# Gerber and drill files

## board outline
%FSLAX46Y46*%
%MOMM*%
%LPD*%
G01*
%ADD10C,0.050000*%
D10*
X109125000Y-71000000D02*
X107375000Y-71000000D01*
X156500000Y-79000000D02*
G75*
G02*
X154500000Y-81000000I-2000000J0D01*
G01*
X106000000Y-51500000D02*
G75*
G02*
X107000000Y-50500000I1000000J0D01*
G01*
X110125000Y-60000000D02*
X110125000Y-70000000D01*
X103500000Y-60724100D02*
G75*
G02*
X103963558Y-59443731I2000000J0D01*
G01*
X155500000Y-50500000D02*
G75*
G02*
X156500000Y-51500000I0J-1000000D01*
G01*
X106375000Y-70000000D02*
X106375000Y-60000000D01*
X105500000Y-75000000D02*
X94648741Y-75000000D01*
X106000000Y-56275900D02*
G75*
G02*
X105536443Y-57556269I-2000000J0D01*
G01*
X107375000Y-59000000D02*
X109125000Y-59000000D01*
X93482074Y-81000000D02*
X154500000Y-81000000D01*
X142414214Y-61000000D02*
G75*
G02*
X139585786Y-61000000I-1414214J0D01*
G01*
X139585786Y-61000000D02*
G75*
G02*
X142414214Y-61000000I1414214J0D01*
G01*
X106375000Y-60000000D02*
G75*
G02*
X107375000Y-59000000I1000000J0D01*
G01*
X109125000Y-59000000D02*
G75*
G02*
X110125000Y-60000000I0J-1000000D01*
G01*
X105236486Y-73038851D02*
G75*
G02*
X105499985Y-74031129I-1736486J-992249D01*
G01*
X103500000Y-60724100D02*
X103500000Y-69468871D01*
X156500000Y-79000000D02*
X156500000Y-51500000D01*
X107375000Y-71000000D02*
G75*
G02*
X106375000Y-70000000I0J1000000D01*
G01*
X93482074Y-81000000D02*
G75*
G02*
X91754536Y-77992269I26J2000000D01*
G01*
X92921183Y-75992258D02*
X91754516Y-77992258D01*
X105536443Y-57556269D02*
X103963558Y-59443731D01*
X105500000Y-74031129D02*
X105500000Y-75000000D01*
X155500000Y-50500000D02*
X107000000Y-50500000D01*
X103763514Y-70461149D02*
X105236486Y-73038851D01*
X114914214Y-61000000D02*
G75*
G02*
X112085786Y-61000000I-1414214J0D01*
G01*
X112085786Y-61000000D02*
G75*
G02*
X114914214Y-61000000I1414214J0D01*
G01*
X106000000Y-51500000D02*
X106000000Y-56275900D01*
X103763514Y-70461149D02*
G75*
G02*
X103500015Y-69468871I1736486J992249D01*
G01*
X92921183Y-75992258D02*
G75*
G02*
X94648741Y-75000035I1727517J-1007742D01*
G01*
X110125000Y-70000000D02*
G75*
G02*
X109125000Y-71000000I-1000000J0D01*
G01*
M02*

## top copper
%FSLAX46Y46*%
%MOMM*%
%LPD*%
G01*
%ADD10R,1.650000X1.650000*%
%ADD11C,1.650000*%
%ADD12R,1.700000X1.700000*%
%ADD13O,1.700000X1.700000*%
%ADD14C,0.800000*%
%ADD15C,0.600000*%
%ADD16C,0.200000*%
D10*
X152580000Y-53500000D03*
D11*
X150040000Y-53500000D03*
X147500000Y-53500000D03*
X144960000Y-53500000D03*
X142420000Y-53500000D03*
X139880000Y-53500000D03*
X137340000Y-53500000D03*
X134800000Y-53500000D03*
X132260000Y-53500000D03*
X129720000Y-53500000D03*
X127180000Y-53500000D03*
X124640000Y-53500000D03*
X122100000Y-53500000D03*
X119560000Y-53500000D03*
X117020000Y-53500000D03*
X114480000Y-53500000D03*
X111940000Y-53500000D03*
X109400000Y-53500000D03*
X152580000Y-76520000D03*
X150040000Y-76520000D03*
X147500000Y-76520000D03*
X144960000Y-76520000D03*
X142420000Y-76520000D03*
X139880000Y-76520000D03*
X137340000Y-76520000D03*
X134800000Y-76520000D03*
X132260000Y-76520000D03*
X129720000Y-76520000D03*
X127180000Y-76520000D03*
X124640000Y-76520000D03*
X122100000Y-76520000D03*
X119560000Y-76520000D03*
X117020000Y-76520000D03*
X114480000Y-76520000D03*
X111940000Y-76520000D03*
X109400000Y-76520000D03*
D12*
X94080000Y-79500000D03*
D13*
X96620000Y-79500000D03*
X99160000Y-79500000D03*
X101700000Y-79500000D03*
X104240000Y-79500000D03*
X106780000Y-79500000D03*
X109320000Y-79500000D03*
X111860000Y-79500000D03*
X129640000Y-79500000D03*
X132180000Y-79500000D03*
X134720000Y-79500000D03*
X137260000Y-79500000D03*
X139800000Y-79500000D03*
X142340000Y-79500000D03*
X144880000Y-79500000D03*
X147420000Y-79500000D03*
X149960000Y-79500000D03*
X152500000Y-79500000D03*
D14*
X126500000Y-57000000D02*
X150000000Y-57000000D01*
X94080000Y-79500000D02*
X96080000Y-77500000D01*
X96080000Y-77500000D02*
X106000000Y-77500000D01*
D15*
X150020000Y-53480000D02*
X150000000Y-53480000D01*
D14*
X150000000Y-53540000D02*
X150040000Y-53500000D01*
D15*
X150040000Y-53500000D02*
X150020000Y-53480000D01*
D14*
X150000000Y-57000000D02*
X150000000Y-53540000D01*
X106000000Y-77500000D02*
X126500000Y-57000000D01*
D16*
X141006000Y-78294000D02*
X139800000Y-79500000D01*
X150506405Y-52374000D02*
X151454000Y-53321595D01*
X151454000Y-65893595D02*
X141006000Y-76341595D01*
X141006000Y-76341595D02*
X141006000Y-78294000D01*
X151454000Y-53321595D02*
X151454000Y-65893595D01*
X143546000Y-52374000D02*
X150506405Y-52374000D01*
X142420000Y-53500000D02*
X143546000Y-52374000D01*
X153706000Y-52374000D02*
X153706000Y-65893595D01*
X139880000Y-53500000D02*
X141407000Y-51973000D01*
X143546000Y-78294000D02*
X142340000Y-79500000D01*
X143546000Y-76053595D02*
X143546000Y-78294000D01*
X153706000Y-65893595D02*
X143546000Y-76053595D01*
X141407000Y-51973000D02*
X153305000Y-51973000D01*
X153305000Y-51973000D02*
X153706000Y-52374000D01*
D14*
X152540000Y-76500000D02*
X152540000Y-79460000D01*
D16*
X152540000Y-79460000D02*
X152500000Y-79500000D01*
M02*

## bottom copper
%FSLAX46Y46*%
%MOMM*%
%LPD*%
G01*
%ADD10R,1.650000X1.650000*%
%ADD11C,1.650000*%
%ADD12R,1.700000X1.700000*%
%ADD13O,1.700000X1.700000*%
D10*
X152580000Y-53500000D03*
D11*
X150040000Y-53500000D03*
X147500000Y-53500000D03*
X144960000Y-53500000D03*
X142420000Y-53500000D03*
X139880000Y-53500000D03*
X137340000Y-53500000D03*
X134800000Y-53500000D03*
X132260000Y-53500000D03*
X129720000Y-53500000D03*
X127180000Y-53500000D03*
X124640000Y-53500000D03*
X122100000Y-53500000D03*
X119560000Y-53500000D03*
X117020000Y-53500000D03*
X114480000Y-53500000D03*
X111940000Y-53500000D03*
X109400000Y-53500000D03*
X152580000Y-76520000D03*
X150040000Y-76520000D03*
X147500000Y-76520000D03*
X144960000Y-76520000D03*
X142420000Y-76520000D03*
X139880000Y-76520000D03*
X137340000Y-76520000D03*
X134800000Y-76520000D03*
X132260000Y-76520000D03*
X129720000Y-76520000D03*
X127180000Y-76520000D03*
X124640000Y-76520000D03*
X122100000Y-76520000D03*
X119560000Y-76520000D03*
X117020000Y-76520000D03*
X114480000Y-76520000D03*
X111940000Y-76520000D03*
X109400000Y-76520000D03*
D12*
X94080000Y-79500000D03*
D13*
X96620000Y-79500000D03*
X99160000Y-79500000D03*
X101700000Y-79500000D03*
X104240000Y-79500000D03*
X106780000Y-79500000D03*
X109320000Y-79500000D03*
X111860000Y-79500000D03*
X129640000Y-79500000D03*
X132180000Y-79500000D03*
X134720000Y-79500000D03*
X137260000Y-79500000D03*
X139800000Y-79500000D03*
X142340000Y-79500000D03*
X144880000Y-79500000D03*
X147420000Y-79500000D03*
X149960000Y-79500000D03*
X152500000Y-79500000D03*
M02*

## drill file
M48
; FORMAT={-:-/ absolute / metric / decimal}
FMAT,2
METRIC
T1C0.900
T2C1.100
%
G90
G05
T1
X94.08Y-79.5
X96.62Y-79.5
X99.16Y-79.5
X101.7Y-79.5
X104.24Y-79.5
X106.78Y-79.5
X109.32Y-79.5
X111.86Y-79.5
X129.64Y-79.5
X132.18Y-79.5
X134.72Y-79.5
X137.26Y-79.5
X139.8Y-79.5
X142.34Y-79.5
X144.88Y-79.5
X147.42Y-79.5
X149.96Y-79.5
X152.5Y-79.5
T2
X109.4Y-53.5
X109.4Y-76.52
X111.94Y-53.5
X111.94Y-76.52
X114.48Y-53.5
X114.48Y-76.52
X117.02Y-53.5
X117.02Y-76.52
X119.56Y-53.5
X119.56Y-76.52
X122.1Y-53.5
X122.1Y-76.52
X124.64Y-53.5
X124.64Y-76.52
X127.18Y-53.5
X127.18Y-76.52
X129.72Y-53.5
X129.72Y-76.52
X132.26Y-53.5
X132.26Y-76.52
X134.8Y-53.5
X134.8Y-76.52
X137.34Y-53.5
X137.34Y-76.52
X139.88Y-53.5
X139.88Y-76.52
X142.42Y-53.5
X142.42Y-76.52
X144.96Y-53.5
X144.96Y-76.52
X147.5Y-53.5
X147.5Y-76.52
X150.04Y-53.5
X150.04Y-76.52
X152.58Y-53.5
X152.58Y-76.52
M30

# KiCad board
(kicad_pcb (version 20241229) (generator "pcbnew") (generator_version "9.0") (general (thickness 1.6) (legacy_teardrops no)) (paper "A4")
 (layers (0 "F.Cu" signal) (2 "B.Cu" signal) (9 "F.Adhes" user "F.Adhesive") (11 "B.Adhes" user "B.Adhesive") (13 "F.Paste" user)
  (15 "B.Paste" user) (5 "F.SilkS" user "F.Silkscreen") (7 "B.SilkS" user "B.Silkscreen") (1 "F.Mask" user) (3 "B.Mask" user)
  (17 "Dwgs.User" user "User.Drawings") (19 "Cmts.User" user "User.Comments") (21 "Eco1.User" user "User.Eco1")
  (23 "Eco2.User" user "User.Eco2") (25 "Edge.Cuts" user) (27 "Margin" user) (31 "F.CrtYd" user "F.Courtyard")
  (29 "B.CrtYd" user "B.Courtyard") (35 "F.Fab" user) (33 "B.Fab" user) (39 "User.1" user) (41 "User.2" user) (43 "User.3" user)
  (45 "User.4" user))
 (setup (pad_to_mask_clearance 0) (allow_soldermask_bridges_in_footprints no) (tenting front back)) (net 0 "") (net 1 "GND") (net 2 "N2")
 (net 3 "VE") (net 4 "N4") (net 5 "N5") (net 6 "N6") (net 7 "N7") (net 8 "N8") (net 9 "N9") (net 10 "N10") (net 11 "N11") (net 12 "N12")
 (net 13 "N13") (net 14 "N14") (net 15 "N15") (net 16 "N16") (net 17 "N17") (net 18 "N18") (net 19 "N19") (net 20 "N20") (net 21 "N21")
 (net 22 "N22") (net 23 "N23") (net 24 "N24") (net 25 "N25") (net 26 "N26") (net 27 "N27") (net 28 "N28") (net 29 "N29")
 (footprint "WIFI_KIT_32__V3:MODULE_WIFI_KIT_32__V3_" (layer "F.Cu") (at 130.18 65.01 -90)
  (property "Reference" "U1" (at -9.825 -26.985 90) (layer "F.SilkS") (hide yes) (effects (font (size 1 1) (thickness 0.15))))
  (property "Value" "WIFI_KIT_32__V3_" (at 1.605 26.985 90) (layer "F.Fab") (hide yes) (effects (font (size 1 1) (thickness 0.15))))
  (pad "J2_1" thru_hole rect (at -11.51 -22.4 270) (size 1.65 1.65) (drill 1.1) (layers "*.Cu" "*.Mask") (remove_unused_layers no)
   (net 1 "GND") (solder_mask_margin 0.102))
  (pad "J2_2" thru_hole circle (at -11.51 -19.86 270) (size 1.65 1.65) (drill 1.1) (layers "*.Cu" "*.Mask") (remove_unused_layers no)
   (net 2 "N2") (solder_mask_margin 0.102))
  (pad "J2_3" thru_hole circle (at -11.51 -17.32 270) (size 1.65 1.65) (drill 1.1) (layers "*.Cu" "*.Mask") (remove_unused_layers no)
   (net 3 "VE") (solder_mask_margin 0.102))
  (pad "J2_4" thru_hole circle (at -11.51 -14.78 270) (size 1.65 1.65) (drill 1.1) (layers "*.Cu" "*.Mask") (remove_unused_layers no)
   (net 3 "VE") (solder_mask_margin 0.102))
  (pad "J2_5" thru_hole circle (at -11.51 -12.24 270) (size 1.65 1.65) (drill 1.1) (layers "*.Cu" "*.Mask") (remove_unused_layers no)
   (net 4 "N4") (solder_mask_margin 0.102))
  (pad "J2_6" thru_hole circle (at -11.51 -9.7 270) (size 1.65 1.65) (drill 1.1) (layers "*.Cu" "*.Mask") (remove_unused_layers no)
   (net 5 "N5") (solder_mask_margin 0.102))
  (pad "J2_7" thru_hole circle (at -11.51 -7.16 270) (size 1.65 1.65) (drill 1.1) (layers "*.Cu" "*.Mask") (remove_unused_layers no)
   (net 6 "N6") (solder_mask_margin 0.102))
  (pad "J2_8" thru_hole circle (at -11.51 -4.62 270) (size 1.65 1.65) (drill 1.1) (layers "*.Cu" "*.Mask") (remove_unused_layers no)
   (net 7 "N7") (solder_mask_margin 0.102))
  (pad "J2_9" thru_hole circle (at -11.51 -2.08 270) (size 1.65 1.65) (drill 1.1) (layers "*.Cu" "*.Mask") (remove_unused_layers no)
   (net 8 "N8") (solder_mask_margin 0.102))
  (pad "J2_10" thru_hole circle (at -11.51 0.46 270) (size 1.65 1.65) (drill 1.1) (layers "*.Cu" "*.Mask") (remove_unused_layers no)
   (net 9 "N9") (solder_mask_margin 0.102))
  (pad "J2_11" thru_hole circle (at -11.51 3 270) (size 1.65 1.65) (drill 1.1) (layers "*.Cu" "*.Mask") (remove_unused_layers no)
   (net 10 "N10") (solder_mask_margin 0.102))
  (pad "J2_12" thru_hole circle (at -11.51 5.54 270) (size 1.65 1.65) (drill 1.1) (layers "*.Cu" "*.Mask") (remove_unused_layers no)
   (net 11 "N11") (solder_mask_margin 0.102))
  (pad "J2_13" thru_hole circle (at -11.51 8.08 270) (size 1.65 1.65) (drill 1.1) (layers "*.Cu" "*.Mask") (remove_unused_layers no)
   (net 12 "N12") (solder_mask_margin 0.102))
  (pad "J2_14" thru_hole circle (at -11.51 10.62 270) (size 1.65 1.65) (drill 1.1) (layers "*.Cu" "*.Mask") (remove_unused_layers no)
   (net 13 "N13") (solder_mask_margin 0.102))
  (pad "J2_15" thru_hole circle (at -11.51 13.16 270) (size 1.65 1.65) (drill 1.1) (layers "*.Cu" "*.Mask") (remove_unused_layers no)
   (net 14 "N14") (solder_mask_margin 0.102))
  (pad "J2_16" thru_hole circle (at -11.51 15.7 270) (size 1.65 1.65) (drill 1.1) (layers "*.Cu" "*.Mask") (remove_unused_layers no)
   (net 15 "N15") (solder_mask_margin 0.102))
  (pad "J2_17" thru_hole circle (at -11.51 18.24 270) (size 1.65 1.65) (drill 1.1) (layers "*.Cu" "*.Mask") (remove_unused_layers no)
   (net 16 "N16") (solder_mask_margin 0.102))
  (pad "J2_18" thru_hole circle (at -11.51 20.78 270) (size 1.65 1.65) (drill 1.1) (layers "*.Cu" "*.Mask") (remove_unused_layers no)
   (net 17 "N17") (solder_mask_margin 0.102))
  (pad "J3_1" thru_hole circle (at 11.51 -22.4 270) (size 1.65 1.65) (drill 1.1) (layers "*.Cu" "*.Mask") (remove_unused_layers no)
   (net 1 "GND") (solder_mask_margin 0.102))
  (pad "J3_2" thru_hole circle (at 11.51 -19.86 270) (size 1.65 1.65) (drill 1.1) (layers "*.Cu" "*.Mask") (remove_unused_layers no)
   (solder_mask_margin 0.102))
  (pad "J3_3" thru_hole circle (at 11.51 -17.32 270) (size 1.65 1.65) (drill 1.1) (layers "*.Cu" "*.Mask") (remove_unused_layers no)
   (solder_mask_margin 0.102))
  (pad "J3_4" thru_hole circle (at 11.51 -14.78 270) (size 1.65 1.65) (drill 1.1) (layers "*.Cu" "*.Mask") (remove_unused_layers no)
   (solder_mask_margin 0.102))
  (pad "J3_5" thru_hole circle (at 11.51 -12.24 270) (size 1.65 1.65) (drill 1.1) (layers "*.Cu" "*.Mask") (remove_unused_layers no)
   (solder_mask_margin 0.102))
  (pad "J3_6" thru_hole circle (at 11.51 -9.7 270) (size 1.65 1.65) (drill 1.1) (layers "*.Cu" "*.Mask") (remove_unused_layers no)
   (solder_mask_margin 0.102))
  (pad "J3_7" thru_hole circle (at 11.51 -7.16 270) (size 1.65 1.65) (drill 1.1) (layers "*.Cu" "*.Mask") (remove_unused_layers no)
   (solder_mask_margin 0.102))
  (pad "J3_8" thru_hole circle (at 11.51 -4.62 270) (size 1.65 1.65) (drill 1.1) (layers "*.Cu" "*.Mask") (remove_unused_layers no)
   (solder_mask_margin 0.102))
  (pad "J3_9" thru_hole circle (at 11.51 -2.08 270) (size 1.65 1.65) (drill 1.1) (layers "*.Cu" "*.Mask") (remove_unused_layers no)
   (solder_mask_margin 0.102))
  (pad "J3_10" thru_hole circle (at 11.51 0.46 270) (size 1.65 1.65) (drill 1.1) (layers "*.Cu" "*.Mask") (remove_unused_layers no)
   (solder_mask_margin 0.102))
  (pad "J3_11" thru_hole circle (at 11.51 3 270) (size 1.65 1.65) (drill 1.1) (layers "*.Cu" "*.Mask") (remove_unused_layers no)
   (solder_mask_margin 0.102))
  (pad "J3_12" thru_hole circle (at 11.51 5.54 270) (size 1.65 1.65) (drill 1.1) (layers "*.Cu" "*.Mask") (remove_unused_layers no)
   (solder_mask_margin 0.102))
  (pad "J3_13" thru_hole circle (at 11.51 8.08 270) (size 1.65 1.65) (drill 1.1) (layers "*.Cu" "*.Mask") (remove_unused_layers no)
   (solder_mask_margin 0.102))
  (pad "J3_14" thru_hole circle (at 11.51 10.62 270) (size 1.65 1.65) (drill 1.1) (layers "*.Cu" "*.Mask") (remove_unused_layers no)
   (solder_mask_margin 0.102))
  (pad "J3_15" thru_hole circle (at 11.51 13.16 270) (size 1.65 1.65) (drill 1.1) (layers "*.Cu" "*.Mask") (remove_unused_layers no)
   (solder_mask_margin 0.102))
  (pad "J3_16" thru_hole circle (at 11.51 15.7 270) (size 1.65 1.65) (drill 1.1) (layers "*.Cu" "*.Mask") (remove_unused_layers no)
   (solder_mask_margin 0.102))
  (pad "J3_17" thru_hole circle (at 11.51 18.24 270) (size 1.65 1.65) (drill 1.1) (layers "*.Cu" "*.Mask") (remove_unused_layers no)
   (solder_mask_margin 0.102))
  (pad "J3_18" thru_hole circle (at 11.51 20.78 270) (size 1.65 1.65) (drill 1.1) (layers "*.Cu" "*.Mask") (remove_unused_layers no)
   (solder_mask_margin 0.102)))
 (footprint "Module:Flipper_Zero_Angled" (layer "F.Cu") (at 94.08 79.5)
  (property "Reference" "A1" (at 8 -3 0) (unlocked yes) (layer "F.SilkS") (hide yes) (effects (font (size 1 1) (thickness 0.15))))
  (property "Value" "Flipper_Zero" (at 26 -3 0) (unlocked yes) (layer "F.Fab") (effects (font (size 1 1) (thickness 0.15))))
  (pad "1" thru_hole rect (at 0 0 90) (size 1.7 1.7) (drill 0.9) (layers "*.Cu" "*.Mask") (remove_unused_layers no) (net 2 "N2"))
  (pad "2" thru_hole oval (at 2.54 0 90) (size 1.7 1.7) (drill 0.9) (layers "*.Cu" "*.Mask") (remove_unused_layers no) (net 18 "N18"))
  (pad "3" thru_hole oval (at 5.08 0 90) (size 1.7 1.7) (drill 0.9) (layers "*.Cu" "*.Mask") (remove_unused_layers no) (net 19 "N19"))
  (pad "4" thru_hole oval (at 7.62 0 90) (size 1.7 1.7) (drill 0.9) (layers "*.Cu" "*.Mask") (remove_unused_layers no) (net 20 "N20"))
  (pad "5" thru_hole oval (at 10.16 0 90) (size 1.7 1.7) (drill 0.9) (layers "*.Cu" "*.Mask") (remove_unused_layers no) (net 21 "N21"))
  (pad "6" thru_hole oval (at 12.7 0 90) (size 1.7 1.7) (drill 0.9) (layers "*.Cu" "*.Mask") (remove_unused_layers no) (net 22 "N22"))
  (pad "7" thru_hole oval (at 15.24 0 90) (size 1.7 1.7) (drill 0.9) (layers "*.Cu" "*.Mask") (remove_unused_layers no) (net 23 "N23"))
  (pad "8" thru_hole oval (at 17.78 0 90) (size 1.7 1.7) (drill 0.9) (layers "*.Cu" "*.Mask") (remove_unused_layers no) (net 1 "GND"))
  (pad "9" thru_hole oval (at 35.56 0 90) (size 1.7 1.7) (drill 0.9) (layers "*.Cu" "*.Mask") (remove_unused_layers no) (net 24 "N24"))
  (pad "10" thru_hole oval (at 38.1 0 90) (size 1.7 1.7) (drill 0.9) (layers "*.Cu" "*.Mask") (remove_unused_layers no) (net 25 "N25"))
  (pad "11" thru_hole oval (at 40.64 0 90) (size 1.7 1.7) (drill 0.9) (layers "*.Cu" "*.Mask") (remove_unused_layers no) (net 1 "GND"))
  (pad "12" thru_hole oval (at 43.18 0 90) (size 1.7 1.7) (drill 0.9) (layers "*.Cu" "*.Mask") (remove_unused_layers no) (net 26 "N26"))
  (pad "13" thru_hole oval (at 45.72 0 90) (size 1.7 1.7) (drill 0.9) (layers "*.Cu" "*.Mask") (remove_unused_layers no) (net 4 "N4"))
  (pad "14" thru_hole oval (at 48.26 0 90) (size 1.7 1.7) (drill 0.9) (layers "*.Cu" "*.Mask") (remove_unused_layers no) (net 5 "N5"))
  (pad "15" thru_hole oval (at 50.8 0 90) (size 1.7 1.7) (drill 0.9) (layers "*.Cu" "*.Mask") (remove_unused_layers no) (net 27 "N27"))
  (pad "16" thru_hole oval (at 53.34 0 90) (size 1.7 1.7) (drill 0.9) (layers "*.Cu" "*.Mask") (remove_unused_layers no) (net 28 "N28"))
  (pad "17" thru_hole oval (at 55.88 0 90) (size 1.7 1.7) (drill 0.9) (layers "*.Cu" "*.Mask") (remove_unused_layers no) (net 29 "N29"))
  (pad "18" thru_hole oval (at 58.42 0 90) (size 1.7 1.7) (drill 0.9) (layers "*.Cu" "*.Mask") (remove_unused_layers no) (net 1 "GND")))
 (gr_line (start 109.125 71) (end 107.375 71) (stroke (width 0.05) (type default)) (layer "Edge.Cuts"))
 (gr_arc (start 156.5 79) (mid 155.914214 80.414214) (end 154.5 81) (stroke (width 0.05) (type default)) (layer "Edge.Cuts"))
 (gr_arc (start 106 51.5) (mid 106.292893 50.792893) (end 107 50.5) (stroke (width 0.05) (type default)) (layer "Edge.Cuts"))
 (gr_line (start 110.125 60) (end 110.125 70) (stroke (width 0.05) (type default)) (layer "Edge.Cuts"))
 (gr_arc (start 103.5 60.7241) (mid 103.619457 60.043249) (end 103.963558 59.443731) (stroke (width 0.05) (type default))
  (layer "Edge.Cuts"))
 (gr_arc (start 155.5 50.5) (mid 156.207107 50.792893) (end 156.5 51.5) (stroke (width 0.05) (type default)) (layer "Edge.Cuts"))
 (gr_line (start 106.375 70) (end 106.375 60) (stroke (width 0.05) (type default)) (layer "Edge.Cuts"))
 (gr_line (start 105.5 75) (end 94.648741 75) (stroke (width 0.05) (type default)) (layer "Edge.Cuts"))
 (gr_arc (start 106 56.2759) (mid 105.880543 56.95675) (end 105.536443 57.556269) (stroke (width 0.05) (type default)) (layer "Edge.Cuts"))
 (gr_line (start 107.375 59) (end 109.125 59) (stroke (width 0.05) (type default)) (layer "Edge.Cuts"))
 (gr_line (start 93.482074 81) (end 154.5 81) (stroke (width 0.05) (type default)) (layer "Edge.Cuts"))
 (gr_circle (center 141 61) (end 142 62) (stroke (width 0.05) (type default)) (fill no) (layer "Edge.Cuts"))
 (gr_arc (start 106.375 60) (mid 106.667893 59.292893) (end 107.375 59) (stroke (width 0.05) (type default)) (layer "Edge.Cuts"))
 (gr_arc (start 109.125 59) (mid 109.832107 59.292893) (end 110.125 60) (stroke (width 0.05) (type default)) (layer "Edge.Cuts"))
 (gr_arc (start 105.236486 73.038851) (mid 105.432999 73.517793) (end 105.5 74.031129) (stroke (width 0.05) (type default))
  (layer "Edge.Cuts"))
 (gr_line (start 103.5 60.7241) (end 103.5 69.468871) (stroke (width 0.05) (type default)) (layer "Edge.Cuts"))
 (gr_line (start 156.5 79) (end 156.5 51.5) (stroke (width 0.05) (type default)) (layer "Edge.Cuts"))
 (gr_arc (start 107.375 71) (mid 106.667893 70.707107) (end 106.375 70) (stroke (width 0.05) (type default)) (layer "Edge.Cuts"))
 (gr_arc (start 93.482074 81) (mid 91.747813 79.996116) (end 91.754516 77.992258) (stroke (width 0.05) (type default)) (layer "Edge.Cuts"))
 (gr_line (start 92.921183 75.992258) (end 91.754516 77.992258) (stroke (width 0.05) (type default)) (layer "Edge.Cuts"))
 (gr_line (start 105.536443 57.556269) (end 103.963558 59.443731) (stroke (width 0.05) (type default)) (layer "Edge.Cuts"))
 (gr_line (start 105.5 74.031129) (end 105.5 75) (stroke (width 0.05) (type default)) (layer "Edge.Cuts"))
 (gr_line (start 155.5 50.5) (end 107 50.5) (stroke (width 0.05) (type default)) (layer "Edge.Cuts"))
 (gr_line (start 103.763514 70.461149) (end 105.236486 73.038851) (stroke (width 0.05) (type default)) (layer "Edge.Cuts"))
 (gr_circle (center 113.5 61) (end 114.5 62) (stroke (width 0.05) (type default)) (fill no) (layer "Edge.Cuts"))
 (gr_line (start 106 51.5) (end 106 56.2759) (stroke (width 0.05) (type default)) (layer "Edge.Cuts"))
 (gr_arc (start 103.763514 70.461149) (mid 103.567001 69.982207) (end 103.5 69.468871) (stroke (width 0.05) (type default))
  (layer "Edge.Cuts"))
 (gr_arc (start 92.921183 75.992258) (mid 93.652619 75.265716) (end 94.648741 75) (stroke (width 0.05) (type default)) (layer "Edge.Cuts"))
 (gr_arc (start 110.125 70) (mid 109.832107 70.707107) (end 109.125 71) (stroke (width 0.05) (type default)) (layer "Edge.Cuts"))
 (segment (start 126.5 57) (end 150 57) (width 0.8) (layer "F.Cu") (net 2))
 (segment (start 94.08 79.5) (end 96.08 77.5) (width 0.8) (layer "F.Cu") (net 2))
 (segment (start 96.08 77.5) (end 106 77.5) (width 0.8) (layer "F.Cu") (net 2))
 (segment (start 150.02 53.48) (end 150 53.48) (width 0.6) (layer "F.Cu") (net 2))
 (segment (start 150 53.54) (end 150.04 53.5) (width 0.8) (layer "F.Cu") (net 2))
 (segment (start 150.04 53.5) (end 150.02 53.48) (width 0.6) (layer "F.Cu") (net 2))
 (segment (start 150 57) (end 150 53.54) (width 0.8) (layer "F.Cu") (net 2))
 (segment (start 106 77.5) (end 126.5 57) (width 0.8) (layer "F.Cu") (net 2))
 (segment (start 141.006 78.294) (end 139.8 79.5) (width 0.2) (layer "F.Cu") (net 4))
 (segment (start 150.506405 52.374) (end 151.454 53.321595) (width 0.2) (layer "F.Cu") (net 4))
 (segment (start 151.454 65.893595) (end 141.006 76.341595) (width 0.2) (layer "F.Cu") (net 4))
 (segment (start 141.006 76.341595) (end 141.006 78.294) (width 0.2) (layer "F.Cu") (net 4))
 (segment (start 151.454 53.321595) (end 151.454 65.893595) (width 0.2) (layer "F.Cu") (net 4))
 (segment (start 143.546 52.374) (end 150.506405 52.374) (width 0.2) (layer "F.Cu") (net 4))
 (segment (start 142.42 53.5) (end 143.546 52.374) (width 0.2) (layer "F.Cu") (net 4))
 (segment (start 153.706 52.374) (end 153.706 65.893595) (width 0.2) (layer "F.Cu") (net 5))
 (segment (start 139.88 53.5) (end 141.407 51.973) (width 0.2) (layer "F.Cu") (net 5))
 (segment (start 143.546 78.294) (end 142.34 79.5) (width 0.2) (layer "F.Cu") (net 5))
 (segment (start 143.546 76.053595) (end 143.546 78.294) (width 0.2) (layer "F.Cu") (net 5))
 (segment (start 153.706 65.893595) (end 143.546 76.053595) (width 0.2) (layer "F.Cu") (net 5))
 (segment (start 141.407 51.973) (end 153.305 51.973) (width 0.2) (layer "F.Cu") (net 5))
 (segment (start 153.305 51.973) (end 153.706 52.374) (width 0.2) (layer "F.Cu") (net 5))
 (segment (start 152.54 76.5) (end 152.54 79.46) (width 0.8) (layer "F.Cu") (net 1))
 (segment (start 152.54 79.46) (end 152.5 79.5) (width 0.2) (layer "F.Cu") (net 1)))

